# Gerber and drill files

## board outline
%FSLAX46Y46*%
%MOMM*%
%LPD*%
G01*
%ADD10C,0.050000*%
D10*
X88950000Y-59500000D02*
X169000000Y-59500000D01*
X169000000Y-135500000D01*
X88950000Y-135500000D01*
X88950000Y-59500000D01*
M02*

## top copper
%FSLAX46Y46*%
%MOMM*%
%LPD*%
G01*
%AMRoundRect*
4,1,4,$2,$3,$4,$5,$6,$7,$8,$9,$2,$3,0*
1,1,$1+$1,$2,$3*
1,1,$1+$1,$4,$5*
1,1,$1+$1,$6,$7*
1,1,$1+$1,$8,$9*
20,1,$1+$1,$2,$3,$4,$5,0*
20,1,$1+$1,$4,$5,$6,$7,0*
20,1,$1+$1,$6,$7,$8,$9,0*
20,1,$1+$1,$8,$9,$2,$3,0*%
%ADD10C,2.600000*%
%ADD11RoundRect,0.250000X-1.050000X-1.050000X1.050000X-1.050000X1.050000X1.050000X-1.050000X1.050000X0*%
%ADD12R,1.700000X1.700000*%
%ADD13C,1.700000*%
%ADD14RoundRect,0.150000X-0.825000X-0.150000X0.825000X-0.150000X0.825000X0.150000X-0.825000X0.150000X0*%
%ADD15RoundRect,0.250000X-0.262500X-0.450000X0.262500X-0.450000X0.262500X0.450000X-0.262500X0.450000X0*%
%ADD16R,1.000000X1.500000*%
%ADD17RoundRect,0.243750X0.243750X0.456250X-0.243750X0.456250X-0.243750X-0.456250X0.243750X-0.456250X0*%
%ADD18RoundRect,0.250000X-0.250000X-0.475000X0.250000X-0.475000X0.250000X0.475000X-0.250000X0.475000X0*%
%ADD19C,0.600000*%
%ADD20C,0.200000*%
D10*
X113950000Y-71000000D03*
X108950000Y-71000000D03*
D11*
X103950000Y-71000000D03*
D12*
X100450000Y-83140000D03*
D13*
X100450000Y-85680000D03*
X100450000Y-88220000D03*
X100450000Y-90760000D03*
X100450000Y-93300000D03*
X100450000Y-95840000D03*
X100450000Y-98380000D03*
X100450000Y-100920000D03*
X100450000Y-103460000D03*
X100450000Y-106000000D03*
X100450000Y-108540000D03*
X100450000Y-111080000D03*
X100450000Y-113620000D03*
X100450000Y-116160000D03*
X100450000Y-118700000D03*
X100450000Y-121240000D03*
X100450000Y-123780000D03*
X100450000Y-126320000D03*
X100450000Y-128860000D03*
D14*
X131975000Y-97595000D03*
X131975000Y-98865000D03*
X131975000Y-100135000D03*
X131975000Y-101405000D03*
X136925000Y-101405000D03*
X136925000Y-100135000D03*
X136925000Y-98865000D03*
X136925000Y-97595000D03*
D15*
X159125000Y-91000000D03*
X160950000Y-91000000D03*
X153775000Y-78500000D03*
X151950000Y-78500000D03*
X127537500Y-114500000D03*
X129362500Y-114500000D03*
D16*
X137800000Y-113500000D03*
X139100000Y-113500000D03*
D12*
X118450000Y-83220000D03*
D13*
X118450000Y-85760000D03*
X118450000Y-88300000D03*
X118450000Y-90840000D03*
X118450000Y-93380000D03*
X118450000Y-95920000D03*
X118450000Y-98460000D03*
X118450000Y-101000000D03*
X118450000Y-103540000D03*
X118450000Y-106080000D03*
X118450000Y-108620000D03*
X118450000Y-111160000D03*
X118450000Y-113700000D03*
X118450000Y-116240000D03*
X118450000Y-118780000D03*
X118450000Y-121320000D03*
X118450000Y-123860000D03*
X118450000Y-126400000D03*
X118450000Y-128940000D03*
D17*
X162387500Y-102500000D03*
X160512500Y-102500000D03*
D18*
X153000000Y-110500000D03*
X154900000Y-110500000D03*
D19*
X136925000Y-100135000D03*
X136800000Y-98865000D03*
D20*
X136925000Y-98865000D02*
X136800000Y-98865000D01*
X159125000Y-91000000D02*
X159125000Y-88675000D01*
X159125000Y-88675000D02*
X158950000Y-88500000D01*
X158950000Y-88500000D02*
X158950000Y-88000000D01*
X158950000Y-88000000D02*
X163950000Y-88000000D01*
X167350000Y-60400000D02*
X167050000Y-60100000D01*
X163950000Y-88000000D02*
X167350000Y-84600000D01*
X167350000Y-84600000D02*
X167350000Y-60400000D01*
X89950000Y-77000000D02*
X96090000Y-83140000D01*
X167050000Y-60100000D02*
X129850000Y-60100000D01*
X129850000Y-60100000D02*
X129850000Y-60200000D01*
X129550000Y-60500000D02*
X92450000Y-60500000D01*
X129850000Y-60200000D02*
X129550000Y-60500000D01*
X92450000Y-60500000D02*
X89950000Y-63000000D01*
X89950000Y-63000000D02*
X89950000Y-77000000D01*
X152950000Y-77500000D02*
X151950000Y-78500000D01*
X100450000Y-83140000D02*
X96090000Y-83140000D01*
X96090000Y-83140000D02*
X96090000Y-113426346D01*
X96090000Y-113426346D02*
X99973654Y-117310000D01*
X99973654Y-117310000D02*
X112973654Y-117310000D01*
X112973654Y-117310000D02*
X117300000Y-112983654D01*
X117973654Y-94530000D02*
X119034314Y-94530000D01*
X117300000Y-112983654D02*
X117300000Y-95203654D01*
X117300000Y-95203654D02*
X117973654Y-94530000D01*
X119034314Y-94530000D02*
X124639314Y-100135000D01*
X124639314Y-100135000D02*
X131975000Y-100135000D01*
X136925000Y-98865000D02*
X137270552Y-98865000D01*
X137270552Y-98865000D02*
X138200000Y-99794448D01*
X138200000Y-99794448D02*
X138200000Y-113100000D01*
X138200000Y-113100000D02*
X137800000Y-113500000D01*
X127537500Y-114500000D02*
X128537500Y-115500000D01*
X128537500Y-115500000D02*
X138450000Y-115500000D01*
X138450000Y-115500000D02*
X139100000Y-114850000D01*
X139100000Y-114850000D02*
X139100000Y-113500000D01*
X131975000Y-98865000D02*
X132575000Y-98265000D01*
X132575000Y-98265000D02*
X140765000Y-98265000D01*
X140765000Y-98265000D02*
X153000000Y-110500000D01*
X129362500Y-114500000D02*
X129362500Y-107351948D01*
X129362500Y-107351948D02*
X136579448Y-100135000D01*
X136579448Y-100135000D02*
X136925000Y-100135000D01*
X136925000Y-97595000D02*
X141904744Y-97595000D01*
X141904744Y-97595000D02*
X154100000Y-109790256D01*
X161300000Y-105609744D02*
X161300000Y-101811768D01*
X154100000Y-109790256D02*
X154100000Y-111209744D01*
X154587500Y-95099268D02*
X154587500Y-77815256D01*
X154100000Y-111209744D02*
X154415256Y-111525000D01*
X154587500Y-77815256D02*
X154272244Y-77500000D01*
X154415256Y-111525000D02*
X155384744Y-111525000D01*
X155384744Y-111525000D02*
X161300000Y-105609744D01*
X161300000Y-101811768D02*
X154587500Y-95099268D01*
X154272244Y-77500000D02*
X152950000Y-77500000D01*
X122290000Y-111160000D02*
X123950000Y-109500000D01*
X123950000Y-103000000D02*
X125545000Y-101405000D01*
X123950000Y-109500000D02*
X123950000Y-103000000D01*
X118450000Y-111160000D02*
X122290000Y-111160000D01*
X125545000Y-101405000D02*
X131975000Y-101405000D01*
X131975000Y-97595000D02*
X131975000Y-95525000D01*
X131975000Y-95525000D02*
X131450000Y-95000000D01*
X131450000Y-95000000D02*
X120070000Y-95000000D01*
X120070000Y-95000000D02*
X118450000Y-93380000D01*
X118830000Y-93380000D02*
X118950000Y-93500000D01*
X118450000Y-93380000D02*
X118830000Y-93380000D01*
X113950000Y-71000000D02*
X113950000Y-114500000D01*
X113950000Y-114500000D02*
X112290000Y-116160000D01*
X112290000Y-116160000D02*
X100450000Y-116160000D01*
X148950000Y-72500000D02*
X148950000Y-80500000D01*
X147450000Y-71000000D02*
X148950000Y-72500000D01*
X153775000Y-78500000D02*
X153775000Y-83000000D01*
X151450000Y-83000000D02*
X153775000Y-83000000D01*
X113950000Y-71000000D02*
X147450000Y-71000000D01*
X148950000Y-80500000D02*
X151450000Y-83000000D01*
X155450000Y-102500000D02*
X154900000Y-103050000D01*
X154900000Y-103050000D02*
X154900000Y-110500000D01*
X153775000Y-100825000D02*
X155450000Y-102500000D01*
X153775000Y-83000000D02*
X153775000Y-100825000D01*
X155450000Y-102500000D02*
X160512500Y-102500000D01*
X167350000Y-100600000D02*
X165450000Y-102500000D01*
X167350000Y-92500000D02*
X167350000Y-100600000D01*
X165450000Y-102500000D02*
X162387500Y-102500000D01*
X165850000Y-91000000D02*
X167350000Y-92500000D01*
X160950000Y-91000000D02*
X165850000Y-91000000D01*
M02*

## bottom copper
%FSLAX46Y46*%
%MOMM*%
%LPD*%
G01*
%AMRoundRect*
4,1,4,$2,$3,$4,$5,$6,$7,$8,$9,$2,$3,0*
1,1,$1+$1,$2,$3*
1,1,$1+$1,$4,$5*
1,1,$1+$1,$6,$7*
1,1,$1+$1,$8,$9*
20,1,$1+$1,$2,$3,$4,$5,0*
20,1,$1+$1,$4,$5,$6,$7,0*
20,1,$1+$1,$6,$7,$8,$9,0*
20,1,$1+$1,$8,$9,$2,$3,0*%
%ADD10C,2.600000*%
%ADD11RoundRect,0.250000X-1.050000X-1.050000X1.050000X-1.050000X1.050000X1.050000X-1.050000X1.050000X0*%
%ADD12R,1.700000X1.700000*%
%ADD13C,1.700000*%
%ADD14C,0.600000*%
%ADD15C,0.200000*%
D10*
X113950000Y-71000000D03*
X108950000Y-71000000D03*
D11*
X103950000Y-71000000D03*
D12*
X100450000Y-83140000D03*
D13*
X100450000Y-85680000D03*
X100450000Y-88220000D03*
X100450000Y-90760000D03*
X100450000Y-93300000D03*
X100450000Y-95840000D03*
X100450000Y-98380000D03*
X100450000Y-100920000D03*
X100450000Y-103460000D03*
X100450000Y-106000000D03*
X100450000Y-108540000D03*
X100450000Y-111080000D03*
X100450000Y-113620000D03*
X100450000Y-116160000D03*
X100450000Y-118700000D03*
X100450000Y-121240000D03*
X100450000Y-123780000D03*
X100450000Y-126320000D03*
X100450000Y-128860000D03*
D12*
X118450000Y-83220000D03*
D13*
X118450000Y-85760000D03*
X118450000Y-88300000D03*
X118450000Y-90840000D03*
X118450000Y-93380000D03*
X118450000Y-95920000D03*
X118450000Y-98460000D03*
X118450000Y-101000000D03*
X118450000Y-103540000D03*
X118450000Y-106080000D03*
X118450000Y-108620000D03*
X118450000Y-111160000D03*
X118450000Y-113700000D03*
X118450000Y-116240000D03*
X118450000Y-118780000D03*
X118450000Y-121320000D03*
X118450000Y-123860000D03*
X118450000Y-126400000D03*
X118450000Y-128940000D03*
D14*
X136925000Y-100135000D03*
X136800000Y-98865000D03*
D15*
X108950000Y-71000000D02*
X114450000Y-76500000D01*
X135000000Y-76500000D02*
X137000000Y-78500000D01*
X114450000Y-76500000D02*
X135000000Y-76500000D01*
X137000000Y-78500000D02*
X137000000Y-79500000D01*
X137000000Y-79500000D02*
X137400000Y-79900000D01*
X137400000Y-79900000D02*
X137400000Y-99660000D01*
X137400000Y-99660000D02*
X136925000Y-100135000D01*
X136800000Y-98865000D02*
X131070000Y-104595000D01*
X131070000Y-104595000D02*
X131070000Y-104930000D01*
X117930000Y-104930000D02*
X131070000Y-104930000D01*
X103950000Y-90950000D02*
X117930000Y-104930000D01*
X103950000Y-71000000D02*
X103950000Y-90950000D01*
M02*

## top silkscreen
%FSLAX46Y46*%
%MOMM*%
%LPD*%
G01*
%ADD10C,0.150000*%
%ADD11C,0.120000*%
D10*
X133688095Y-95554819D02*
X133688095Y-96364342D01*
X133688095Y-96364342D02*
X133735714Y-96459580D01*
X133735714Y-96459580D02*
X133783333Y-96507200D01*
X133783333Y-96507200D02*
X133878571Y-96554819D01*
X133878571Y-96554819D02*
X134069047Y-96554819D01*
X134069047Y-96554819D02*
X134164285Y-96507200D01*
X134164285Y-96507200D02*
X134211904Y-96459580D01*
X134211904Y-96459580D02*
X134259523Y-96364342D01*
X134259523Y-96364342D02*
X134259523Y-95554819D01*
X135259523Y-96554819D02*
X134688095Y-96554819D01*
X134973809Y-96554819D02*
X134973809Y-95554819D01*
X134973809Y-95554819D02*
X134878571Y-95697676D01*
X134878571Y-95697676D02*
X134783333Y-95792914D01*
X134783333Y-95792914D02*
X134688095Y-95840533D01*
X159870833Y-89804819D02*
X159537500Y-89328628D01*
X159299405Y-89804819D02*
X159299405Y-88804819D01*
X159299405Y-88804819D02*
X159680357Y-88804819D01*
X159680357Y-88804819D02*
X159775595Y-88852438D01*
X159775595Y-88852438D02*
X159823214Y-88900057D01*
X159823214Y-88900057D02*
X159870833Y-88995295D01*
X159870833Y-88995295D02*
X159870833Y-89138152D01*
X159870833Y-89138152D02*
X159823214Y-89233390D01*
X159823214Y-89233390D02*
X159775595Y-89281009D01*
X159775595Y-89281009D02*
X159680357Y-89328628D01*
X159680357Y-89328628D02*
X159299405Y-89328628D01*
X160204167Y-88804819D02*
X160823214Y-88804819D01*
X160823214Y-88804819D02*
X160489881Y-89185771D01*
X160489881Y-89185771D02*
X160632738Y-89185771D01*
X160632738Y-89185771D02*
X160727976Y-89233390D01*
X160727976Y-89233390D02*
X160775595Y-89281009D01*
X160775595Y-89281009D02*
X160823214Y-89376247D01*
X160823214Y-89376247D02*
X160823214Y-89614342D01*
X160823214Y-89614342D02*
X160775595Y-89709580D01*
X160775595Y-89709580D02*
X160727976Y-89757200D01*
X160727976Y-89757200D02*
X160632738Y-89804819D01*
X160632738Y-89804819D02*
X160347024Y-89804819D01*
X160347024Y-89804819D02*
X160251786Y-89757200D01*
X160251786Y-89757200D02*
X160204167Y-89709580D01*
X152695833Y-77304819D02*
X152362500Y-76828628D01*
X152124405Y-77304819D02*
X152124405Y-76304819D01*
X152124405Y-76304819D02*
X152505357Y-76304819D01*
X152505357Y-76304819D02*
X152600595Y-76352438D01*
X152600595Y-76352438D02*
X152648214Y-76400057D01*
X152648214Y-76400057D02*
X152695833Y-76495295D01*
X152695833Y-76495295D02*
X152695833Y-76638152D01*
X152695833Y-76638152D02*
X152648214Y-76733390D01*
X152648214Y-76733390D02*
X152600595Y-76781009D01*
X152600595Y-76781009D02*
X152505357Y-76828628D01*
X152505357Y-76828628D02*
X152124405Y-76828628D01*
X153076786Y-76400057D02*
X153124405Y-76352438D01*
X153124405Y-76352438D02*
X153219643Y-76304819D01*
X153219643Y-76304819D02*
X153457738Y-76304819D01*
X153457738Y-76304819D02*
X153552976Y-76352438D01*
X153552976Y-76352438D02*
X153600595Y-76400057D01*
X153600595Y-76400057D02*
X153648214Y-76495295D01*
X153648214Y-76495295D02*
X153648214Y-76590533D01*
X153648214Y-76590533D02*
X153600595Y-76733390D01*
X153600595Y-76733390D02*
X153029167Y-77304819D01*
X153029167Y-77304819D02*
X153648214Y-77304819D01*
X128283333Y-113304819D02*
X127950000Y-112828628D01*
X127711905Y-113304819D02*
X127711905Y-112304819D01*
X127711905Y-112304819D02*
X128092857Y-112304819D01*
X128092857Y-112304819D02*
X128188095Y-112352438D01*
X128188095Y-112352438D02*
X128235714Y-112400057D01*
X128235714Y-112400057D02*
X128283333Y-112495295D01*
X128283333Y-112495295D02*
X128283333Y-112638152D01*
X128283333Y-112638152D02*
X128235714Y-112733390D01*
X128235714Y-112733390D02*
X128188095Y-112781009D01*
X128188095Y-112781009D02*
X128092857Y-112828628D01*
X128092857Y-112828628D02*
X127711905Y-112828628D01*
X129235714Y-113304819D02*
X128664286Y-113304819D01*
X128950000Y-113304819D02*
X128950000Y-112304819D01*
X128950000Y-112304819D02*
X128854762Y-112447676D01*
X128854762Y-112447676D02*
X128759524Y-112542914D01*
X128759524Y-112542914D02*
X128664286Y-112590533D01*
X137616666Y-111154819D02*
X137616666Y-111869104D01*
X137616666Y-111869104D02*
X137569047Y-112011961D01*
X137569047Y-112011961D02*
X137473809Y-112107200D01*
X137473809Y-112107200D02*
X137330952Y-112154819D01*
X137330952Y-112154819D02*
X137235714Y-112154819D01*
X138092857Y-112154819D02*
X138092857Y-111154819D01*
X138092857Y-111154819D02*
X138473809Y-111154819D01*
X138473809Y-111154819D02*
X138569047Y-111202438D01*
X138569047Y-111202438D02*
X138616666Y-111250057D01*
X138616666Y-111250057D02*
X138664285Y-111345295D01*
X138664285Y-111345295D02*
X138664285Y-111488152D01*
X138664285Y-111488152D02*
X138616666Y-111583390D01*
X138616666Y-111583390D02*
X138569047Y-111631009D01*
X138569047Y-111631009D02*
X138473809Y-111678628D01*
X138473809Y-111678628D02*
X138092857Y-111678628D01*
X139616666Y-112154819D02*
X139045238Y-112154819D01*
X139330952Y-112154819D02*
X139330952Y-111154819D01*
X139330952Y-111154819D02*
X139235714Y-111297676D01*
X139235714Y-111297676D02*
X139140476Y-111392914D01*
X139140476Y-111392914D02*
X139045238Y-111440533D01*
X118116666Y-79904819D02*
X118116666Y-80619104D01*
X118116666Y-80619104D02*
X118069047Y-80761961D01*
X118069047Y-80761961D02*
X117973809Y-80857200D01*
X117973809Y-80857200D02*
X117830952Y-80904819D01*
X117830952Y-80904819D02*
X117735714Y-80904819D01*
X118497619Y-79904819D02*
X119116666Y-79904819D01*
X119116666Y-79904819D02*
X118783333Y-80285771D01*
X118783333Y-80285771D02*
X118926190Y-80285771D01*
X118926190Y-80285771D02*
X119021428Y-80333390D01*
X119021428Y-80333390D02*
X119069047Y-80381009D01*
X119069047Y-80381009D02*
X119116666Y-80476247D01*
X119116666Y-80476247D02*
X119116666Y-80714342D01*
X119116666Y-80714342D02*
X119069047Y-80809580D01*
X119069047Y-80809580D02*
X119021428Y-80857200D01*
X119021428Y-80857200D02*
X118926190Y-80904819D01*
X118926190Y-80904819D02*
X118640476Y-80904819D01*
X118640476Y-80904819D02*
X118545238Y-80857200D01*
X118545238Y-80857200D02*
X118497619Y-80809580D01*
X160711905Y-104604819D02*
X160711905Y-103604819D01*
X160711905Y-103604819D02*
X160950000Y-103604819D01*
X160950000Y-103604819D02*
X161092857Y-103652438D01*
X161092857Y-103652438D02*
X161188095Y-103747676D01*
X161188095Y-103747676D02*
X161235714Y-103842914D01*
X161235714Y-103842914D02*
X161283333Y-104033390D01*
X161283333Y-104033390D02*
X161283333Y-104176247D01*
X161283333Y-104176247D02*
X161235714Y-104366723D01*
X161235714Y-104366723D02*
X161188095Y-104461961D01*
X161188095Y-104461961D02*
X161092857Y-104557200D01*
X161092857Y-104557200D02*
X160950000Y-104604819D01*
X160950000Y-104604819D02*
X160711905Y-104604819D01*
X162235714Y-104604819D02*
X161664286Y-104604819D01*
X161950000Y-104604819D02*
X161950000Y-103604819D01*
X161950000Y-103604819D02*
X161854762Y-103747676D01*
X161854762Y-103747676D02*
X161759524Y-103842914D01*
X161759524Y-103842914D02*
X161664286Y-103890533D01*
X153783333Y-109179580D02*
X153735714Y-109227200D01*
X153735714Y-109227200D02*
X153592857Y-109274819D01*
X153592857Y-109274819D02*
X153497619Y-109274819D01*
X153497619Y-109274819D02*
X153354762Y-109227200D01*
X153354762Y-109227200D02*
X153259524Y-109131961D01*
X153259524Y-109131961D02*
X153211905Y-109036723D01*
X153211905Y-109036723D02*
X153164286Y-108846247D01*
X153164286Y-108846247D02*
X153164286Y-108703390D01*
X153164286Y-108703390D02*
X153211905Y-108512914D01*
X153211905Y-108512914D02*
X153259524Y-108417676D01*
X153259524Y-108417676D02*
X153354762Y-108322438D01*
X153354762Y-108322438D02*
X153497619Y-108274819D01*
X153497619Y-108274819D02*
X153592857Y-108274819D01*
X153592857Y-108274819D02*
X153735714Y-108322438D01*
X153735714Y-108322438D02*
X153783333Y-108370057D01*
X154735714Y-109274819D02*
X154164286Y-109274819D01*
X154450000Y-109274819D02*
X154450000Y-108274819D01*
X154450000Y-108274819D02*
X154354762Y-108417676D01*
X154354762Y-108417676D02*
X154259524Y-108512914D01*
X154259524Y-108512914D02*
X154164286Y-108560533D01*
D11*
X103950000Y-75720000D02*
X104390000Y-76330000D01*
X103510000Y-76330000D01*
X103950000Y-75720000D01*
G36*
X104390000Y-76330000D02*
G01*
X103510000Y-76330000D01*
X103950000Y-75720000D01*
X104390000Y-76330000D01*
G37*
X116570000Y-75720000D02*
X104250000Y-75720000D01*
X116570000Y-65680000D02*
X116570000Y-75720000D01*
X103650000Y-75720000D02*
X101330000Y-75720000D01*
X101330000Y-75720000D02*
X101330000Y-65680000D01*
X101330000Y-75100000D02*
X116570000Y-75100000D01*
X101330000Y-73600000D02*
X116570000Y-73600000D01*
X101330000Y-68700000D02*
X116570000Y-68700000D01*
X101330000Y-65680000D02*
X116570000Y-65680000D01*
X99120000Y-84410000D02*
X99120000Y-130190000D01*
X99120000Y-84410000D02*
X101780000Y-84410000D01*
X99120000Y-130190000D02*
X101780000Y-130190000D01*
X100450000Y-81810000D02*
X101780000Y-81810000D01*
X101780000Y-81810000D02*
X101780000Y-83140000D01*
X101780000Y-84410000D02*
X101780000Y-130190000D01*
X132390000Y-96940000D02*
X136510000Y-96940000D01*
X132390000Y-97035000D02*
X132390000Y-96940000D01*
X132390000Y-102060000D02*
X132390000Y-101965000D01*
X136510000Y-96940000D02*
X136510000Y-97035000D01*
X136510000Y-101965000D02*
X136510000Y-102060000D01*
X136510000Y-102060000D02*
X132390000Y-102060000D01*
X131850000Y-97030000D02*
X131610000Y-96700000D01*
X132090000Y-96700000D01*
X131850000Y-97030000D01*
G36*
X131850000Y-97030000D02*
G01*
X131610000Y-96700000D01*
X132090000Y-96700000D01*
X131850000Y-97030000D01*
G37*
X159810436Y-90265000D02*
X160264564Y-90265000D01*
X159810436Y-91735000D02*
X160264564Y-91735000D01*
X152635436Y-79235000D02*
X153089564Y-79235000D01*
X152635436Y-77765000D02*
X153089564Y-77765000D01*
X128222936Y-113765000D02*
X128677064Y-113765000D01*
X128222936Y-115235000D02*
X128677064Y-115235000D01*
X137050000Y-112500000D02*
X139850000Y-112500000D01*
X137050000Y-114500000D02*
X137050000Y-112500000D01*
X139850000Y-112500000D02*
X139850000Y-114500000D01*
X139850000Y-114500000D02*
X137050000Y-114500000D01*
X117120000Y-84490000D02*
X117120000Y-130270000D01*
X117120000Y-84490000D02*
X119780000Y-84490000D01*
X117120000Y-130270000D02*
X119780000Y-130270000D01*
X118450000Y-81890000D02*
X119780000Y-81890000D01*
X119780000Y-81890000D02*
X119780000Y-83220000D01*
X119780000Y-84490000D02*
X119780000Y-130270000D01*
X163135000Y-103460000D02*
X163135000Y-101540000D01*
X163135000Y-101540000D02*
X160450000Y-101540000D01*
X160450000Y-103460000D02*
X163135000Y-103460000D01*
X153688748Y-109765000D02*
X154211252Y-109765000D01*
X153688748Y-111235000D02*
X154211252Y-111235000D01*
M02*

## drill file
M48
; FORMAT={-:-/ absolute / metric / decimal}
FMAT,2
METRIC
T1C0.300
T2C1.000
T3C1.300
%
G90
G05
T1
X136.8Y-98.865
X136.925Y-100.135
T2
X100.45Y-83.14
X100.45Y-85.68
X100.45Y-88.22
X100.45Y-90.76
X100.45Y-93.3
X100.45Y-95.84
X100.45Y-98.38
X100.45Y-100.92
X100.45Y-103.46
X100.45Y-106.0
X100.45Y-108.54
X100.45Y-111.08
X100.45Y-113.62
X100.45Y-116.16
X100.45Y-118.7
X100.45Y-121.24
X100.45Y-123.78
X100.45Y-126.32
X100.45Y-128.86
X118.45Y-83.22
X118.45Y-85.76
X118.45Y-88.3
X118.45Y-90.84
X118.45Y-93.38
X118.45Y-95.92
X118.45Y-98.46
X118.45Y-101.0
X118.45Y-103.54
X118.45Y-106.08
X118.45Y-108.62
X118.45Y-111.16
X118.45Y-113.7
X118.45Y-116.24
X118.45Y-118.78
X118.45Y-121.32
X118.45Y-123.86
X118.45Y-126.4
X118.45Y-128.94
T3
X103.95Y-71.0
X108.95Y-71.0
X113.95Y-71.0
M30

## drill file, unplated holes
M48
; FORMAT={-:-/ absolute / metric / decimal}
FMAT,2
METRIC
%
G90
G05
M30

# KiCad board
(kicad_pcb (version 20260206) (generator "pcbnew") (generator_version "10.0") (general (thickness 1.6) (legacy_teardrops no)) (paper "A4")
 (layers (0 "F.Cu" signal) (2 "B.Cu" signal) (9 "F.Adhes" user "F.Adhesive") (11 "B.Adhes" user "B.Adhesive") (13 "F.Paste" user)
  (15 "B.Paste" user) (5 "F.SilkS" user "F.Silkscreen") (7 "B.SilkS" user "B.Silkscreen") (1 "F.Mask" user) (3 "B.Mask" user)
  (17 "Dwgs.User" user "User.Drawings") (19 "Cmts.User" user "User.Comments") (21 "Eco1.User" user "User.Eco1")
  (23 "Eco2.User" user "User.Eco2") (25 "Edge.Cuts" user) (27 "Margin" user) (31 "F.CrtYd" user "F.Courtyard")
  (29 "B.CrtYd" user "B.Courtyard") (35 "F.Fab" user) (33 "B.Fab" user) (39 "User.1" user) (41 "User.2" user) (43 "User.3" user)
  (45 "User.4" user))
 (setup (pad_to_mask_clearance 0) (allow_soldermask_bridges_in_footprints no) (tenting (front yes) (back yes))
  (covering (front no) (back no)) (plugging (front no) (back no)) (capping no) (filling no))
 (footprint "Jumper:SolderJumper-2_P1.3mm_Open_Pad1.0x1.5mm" (layer "F.Cu") (at 138.45 113.5)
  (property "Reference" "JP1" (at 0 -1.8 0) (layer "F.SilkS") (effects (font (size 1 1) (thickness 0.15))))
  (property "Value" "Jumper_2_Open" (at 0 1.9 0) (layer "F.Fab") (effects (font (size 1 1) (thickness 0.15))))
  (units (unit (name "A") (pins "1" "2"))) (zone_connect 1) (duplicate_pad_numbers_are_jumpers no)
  (fp_line (start -1.4 -1) (end 1.4 -1) (stroke (width 0.12) (type solid)) (layer "F.SilkS"))
  (fp_line (start -1.4 1) (end -1.4 -1) (stroke (width 0.12) (type solid)) (layer "F.SilkS"))
  (fp_line (start 1.4 -1) (end 1.4 1) (stroke (width 0.12) (type solid)) (layer "F.SilkS"))
  (fp_line (start 1.4 1) (end -1.4 1) (stroke (width 0.12) (type solid)) (layer "F.SilkS"))
  (pad "1" smd rect (at -0.65 0) (size 1 1.5) (layers "F.Cu" "F.Mask") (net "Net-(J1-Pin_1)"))
  (pad "2" smd rect (at 0.65 0) (size 1 1.5) (layers "F.Cu" "F.Mask") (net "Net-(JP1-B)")))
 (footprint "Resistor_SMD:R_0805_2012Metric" (layer "F.Cu") (at 152.8625 78.5)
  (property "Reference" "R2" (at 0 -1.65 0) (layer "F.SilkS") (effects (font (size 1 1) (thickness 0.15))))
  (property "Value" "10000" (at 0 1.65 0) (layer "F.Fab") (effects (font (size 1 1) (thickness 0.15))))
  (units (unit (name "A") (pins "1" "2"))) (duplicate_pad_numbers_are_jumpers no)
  (fp_line (start -0.227064 -0.735) (end 0.227064 -0.735) (stroke (width 0.12) (type solid)) (layer "F.SilkS"))
  (fp_line (start -0.227064 0.735) (end 0.227064 0.735) (stroke (width 0.12) (type solid)) (layer "F.SilkS"))
  (pad "1" smd roundrect (at -0.9125 0) (size 1.025 1.4) (layers "F.Cu" "F.Mask" "F.Paste") (roundrect_rratio 0.243902) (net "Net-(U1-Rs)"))
  (pad "2" smd roundrect (at 0.9125 0) (size 1.025 1.4) (layers "F.Cu" "F.Mask" "F.Paste") (roundrect_rratio 0.243902) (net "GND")))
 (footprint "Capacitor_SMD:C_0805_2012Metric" (layer "F.Cu") (at 153.95 110.5)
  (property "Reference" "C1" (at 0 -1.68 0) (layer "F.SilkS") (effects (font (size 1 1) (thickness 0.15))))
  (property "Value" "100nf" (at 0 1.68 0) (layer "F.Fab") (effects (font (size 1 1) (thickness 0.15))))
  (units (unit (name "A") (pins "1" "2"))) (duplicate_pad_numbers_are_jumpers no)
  (fp_line (start -0.261252 -0.735) (end 0.261252 -0.735) (stroke (width 0.12) (type solid)) (layer "F.SilkS"))
  (fp_line (start -0.261252 0.735) (end 0.261252 0.735) (stroke (width 0.12) (type solid)) (layer "F.SilkS"))
  (pad "1" smd roundrect (at -0.95 0) (size 1 1.45) (layers "F.Cu" "F.Mask" "F.Paste") (roundrect_rratio 0.25) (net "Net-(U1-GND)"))
  (pad "2" smd roundrect (at 0.95 0) (size 1 1.45) (layers "F.Cu" "F.Mask" "F.Paste") (roundrect_rratio 0.25) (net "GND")))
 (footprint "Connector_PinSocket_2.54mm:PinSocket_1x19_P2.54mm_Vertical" (layer "F.Cu") (at 100.45 83.14)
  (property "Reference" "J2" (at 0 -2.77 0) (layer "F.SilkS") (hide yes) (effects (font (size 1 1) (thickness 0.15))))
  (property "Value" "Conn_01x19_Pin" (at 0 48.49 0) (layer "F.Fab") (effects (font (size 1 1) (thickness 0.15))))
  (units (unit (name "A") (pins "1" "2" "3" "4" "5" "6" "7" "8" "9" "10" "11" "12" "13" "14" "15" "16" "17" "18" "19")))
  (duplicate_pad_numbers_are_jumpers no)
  (fp_line (start -1.33 1.27) (end -1.33 47.05) (stroke (width 0.12) (type solid)) (layer "F.SilkS"))
  (fp_line (start -1.33 1.27) (end 1.33 1.27) (stroke (width 0.12) (type solid)) (layer "F.SilkS"))
  (fp_line (start -1.33 47.05) (end 1.33 47.05) (stroke (width 0.12) (type solid)) (layer "F.SilkS"))
  (fp_line (start 0 -1.33) (end 1.33 -1.33) (stroke (width 0.12) (type solid)) (layer "F.SilkS"))
  (fp_line (start 1.33 -1.33) (end 1.33 0) (stroke (width 0.12) (type solid)) (layer "F.SilkS"))
  (fp_line (start 1.33 1.27) (end 1.33 47.05) (stroke (width 0.12) (type solid)) (layer "F.SilkS"))
  (pad "1" thru_hole rect (at 0 0) (size 1.7 1.7) (drill 1) (layers "*.Cu" "*.Mask") (remove_unused_layers no) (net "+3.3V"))
  (pad "2" thru_hole circle (at 0 2.54) (size 1.7 1.7) (drill 1) (layers "*.Cu" "*.Mask") (remove_unused_layers no)
   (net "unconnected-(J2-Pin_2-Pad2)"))
  (pad "3" thru_hole circle (at 0 5.08) (size 1.7 1.7) (drill 1) (layers "*.Cu" "*.Mask") (remove_unused_layers no)
   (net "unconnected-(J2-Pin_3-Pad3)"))
  (pad "4" thru_hole circle (at 0 7.62) (size 1.7 1.7) (drill 1) (layers "*.Cu" "*.Mask") (remove_unused_layers no)
   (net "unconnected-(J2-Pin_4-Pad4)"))
  (pad "5" thru_hole circle (at 0 10.16) (size 1.7 1.7) (drill 1) (layers "*.Cu" "*.Mask") (remove_unused_layers no)
   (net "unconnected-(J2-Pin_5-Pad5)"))
  (pad "6" thru_hole circle (at 0 12.7) (size 1.7 1.7) (drill 1) (layers "*.Cu" "*.Mask") (remove_unused_layers no)
   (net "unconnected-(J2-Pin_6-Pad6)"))
  (pad "7" thru_hole circle (at 0 15.24) (size 1.7 1.7) (drill 1) (layers "*.Cu" "*.Mask") (remove_unused_layers no)
   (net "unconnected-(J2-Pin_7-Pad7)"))
  (pad "8" thru_hole circle (at 0 17.78) (size 1.7 1.7) (drill 1) (layers "*.Cu" "*.Mask") (remove_unused_layers no)
   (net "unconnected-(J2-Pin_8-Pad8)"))
  (pad "9" thru_hole circle (at 0 20.32) (size 1.7 1.7) (drill 1) (layers "*.Cu" "*.Mask") (remove_unused_layers no)
   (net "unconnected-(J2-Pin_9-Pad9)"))
  (pad "10" thru_hole circle (at 0 22.86) (size 1.7 1.7) (drill 1) (layers "*.Cu" "*.Mask") (remove_unused_layers no)
   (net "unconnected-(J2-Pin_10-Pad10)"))
  (pad "11" thru_hole circle (at 0 25.4) (size 1.7 1.7) (drill 1) (layers "*.Cu" "*.Mask") (remove_unused_layers no)
   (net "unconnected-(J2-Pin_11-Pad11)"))
  (pad "12" thru_hole circle (at 0 27.94) (size 1.7 1.7) (drill 1) (layers "*.Cu" "*.Mask") (remove_unused_layers no)
   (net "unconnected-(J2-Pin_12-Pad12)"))
  (pad "13" thru_hole circle (at 0 30.48) (size 1.7 1.7) (drill 1) (layers "*.Cu" "*.Mask") (remove_unused_layers no)
   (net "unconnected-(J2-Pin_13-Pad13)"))
  (pad "14" thru_hole circle (at 0 33.02) (size 1.7 1.7) (drill 1) (layers "*.Cu" "*.Mask") (remove_unused_layers no) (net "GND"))
  (pad "15" thru_hole circle (at 0 35.56) (size 1.7 1.7) (drill 1) (layers "*.Cu" "*.Mask") (remove_unused_layers no)
   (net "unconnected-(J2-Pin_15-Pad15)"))
  (pad "16" thru_hole circle (at 0 38.1) (size 1.7 1.7) (drill 1) (layers "*.Cu" "*.Mask") (remove_unused_layers no)
   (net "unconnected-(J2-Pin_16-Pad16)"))
  (pad "17" thru_hole circle (at 0 40.64) (size 1.7 1.7) (drill 1) (layers "*.Cu" "*.Mask") (remove_unused_layers no)
   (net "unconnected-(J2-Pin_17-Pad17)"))
  (pad "18" thru_hole circle (at 0 43.18) (size 1.7 1.7) (drill 1) (layers "*.Cu" "*.Mask") (remove_unused_layers no)
   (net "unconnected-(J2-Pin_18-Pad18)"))
  (pad "19" thru_hole circle (at 0 45.72) (size 1.7 1.7) (drill 1) (layers "*.Cu" "*.Mask") (remove_unused_layers no)
   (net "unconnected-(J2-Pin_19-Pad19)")))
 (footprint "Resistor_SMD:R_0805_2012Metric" (layer "F.Cu") (at 128.45 114.5)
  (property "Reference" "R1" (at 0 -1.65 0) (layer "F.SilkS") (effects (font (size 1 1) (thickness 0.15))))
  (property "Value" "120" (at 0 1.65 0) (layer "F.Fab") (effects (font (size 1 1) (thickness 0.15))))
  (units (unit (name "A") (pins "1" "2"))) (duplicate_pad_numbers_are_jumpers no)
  (fp_line (start -0.227064 -0.735) (end 0.227064 -0.735) (stroke (width 0.12) (type solid)) (layer "F.SilkS"))
  (fp_line (start -0.227064 0.735) (end 0.227064 0.735) (stroke (width 0.12) (type solid)) (layer "F.SilkS"))
  (pad "1" smd roundrect (at -0.9125 0) (size 1.025 1.4) (layers "F.Cu" "F.Mask" "F.Paste") (roundrect_rratio 0.243902) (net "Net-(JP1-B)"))
  (pad "2" smd roundrect (at 0.9125 0) (size 1.025 1.4) (layers "F.Cu" "F.Mask" "F.Paste") (roundrect_rratio 0.243902)
   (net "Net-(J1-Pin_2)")))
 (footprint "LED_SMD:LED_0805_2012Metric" (layer "F.Cu") (at 161.45 102.5 180)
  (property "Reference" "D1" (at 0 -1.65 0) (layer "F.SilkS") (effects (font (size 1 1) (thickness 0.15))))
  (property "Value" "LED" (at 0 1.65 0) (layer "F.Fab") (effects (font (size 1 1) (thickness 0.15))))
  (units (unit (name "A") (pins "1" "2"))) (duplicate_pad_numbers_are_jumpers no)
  (fp_line (start 1 -0.96) (end -1.685 -0.96) (stroke (width 0.12) (type solid)) (layer "F.SilkS"))
  (fp_line (start -1.685 0.96) (end 1 0.96) (stroke (width 0.12) (type solid)) (layer "F.SilkS"))
  (fp_line (start -1.685 -0.96) (end -1.685 0.96) (stroke (width 0.12) (type solid)) (layer "F.SilkS"))
  (pad "1" smd roundrect (at -0.9375 0 180) (size 0.975 1.4) (layers "F.Cu" "F.Mask" "F.Paste") (roundrect_rratio 0.25) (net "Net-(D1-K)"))
  (pad "2" smd roundrect (at 0.9375 0 180) (size 0.975 1.4) (layers "F.Cu" "F.Mask" "F.Paste") (roundrect_rratio 0.25) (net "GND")))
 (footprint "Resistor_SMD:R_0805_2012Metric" (layer "F.Cu") (at 160.0375 91)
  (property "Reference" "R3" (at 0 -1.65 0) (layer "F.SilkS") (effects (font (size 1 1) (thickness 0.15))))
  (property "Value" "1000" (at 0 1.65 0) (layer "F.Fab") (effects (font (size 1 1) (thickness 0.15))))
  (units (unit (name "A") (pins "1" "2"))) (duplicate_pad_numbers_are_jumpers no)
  (fp_line (start -0.227064 -0.735) (end 0.227064 -0.735) (stroke (width 0.12) (type solid)) (layer "F.SilkS"))
  (fp_line (start -0.227064 0.735) (end 0.227064 0.735) (stroke (width 0.12) (type solid)) (layer "F.SilkS"))
  (pad "1" smd roundrect (at -0.9125 0) (size 1.025 1.4) (layers "F.Cu" "F.Mask" "F.Paste") (roundrect_rratio 0.243902) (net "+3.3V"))
  (pad "2" smd roundrect (at 0.9125 0) (size 1.025 1.4) (layers "F.Cu" "F.Mask" "F.Paste") (roundrect_rratio 0.243902) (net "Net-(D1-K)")))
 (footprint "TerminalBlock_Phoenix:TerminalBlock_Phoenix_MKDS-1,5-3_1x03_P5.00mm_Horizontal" (layer "F.Cu") (at 103.95 71)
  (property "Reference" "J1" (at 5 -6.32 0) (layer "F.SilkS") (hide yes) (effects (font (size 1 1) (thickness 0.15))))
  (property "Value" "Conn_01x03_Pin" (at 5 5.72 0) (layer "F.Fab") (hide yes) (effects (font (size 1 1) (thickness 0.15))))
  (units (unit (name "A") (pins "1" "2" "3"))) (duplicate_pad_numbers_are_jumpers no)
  (fp_line (start -2.62 -5.32) (end 12.62 -5.32) (stroke (width 0.12) (type solid)) (layer "F.SilkS"))
  (fp_line (start -2.62 -2.3) (end 12.62 -2.3) (stroke (width 0.12) (type solid)) (layer "F.SilkS"))
  (fp_line (start -2.62 2.6) (end 12.62 2.6) (stroke (width 0.12) (type solid)) (layer "F.SilkS"))
  (fp_line (start -2.62 4.1) (end 12.62 4.1) (stroke (width 0.12) (type solid)) (layer "F.SilkS"))
  (fp_line (start -2.62 4.72) (end -2.62 -5.32) (stroke (width 0.12) (type solid)) (layer "F.SilkS"))
  (fp_line (start -0.3 4.72) (end -2.62 4.72) (stroke (width 0.12) (type solid)) (layer "F.SilkS"))
  (fp_line (start 12.62 -5.32) (end 12.62 4.72) (stroke (width 0.12) (type solid)) (layer "F.SilkS"))
  (fp_line (start 12.62 4.72) (end 0.3 4.72) (stroke (width 0.12) (type solid)) (layer "F.SilkS"))
  (fp_poly (pts (xy 0 4.72) (xy 0.44 5.33) (xy -0.44 5.33)) (stroke (width 0.12) (type solid)) (fill yes) (layer "F.SilkS"))
  (pad "1" thru_hole roundrect (at 0 0) (size 2.6 2.6) (drill 1.3) (layers "*.Cu" "*.Mask") (remove_unused_layers no)
   (roundrect_rratio 0.096154) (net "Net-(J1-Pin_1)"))
  (pad "2" thru_hole circle (at 5 0) (size 2.6 2.6) (drill 1.3) (layers "*.Cu" "*.Mask") (remove_unused_layers no) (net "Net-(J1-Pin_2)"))
  (pad "3" thru_hole circle (at 10 0) (size 2.6 2.6) (drill 1.3) (layers "*.Cu" "*.Mask") (remove_unused_layers no) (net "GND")))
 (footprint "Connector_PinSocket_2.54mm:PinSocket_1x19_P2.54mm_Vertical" (layer "F.Cu") (at 118.45 83.22)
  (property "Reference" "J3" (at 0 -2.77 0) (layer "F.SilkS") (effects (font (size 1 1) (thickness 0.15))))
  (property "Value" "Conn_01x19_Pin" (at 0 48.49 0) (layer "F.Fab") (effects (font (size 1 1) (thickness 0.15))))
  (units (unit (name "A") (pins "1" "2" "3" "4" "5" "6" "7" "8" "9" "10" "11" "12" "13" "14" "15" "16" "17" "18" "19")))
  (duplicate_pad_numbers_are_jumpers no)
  (fp_line (start -1.33 1.27) (end -1.33 47.05) (stroke (width 0.12) (type solid)) (layer "F.SilkS"))
  (fp_line (start -1.33 1.27) (end 1.33 1.27) (stroke (width 0.12) (type solid)) (layer "F.SilkS"))
  (fp_line (start -1.33 47.05) (end 1.33 47.05) (stroke (width 0.12) (type solid)) (layer "F.SilkS"))
  (fp_line (start 0 -1.33) (end 1.33 -1.33) (stroke (width 0.12) (type solid)) (layer "F.SilkS"))
  (fp_line (start 1.33 -1.33) (end 1.33 0) (stroke (width 0.12) (type solid)) (layer "F.SilkS"))
  (fp_line (start 1.33 1.27) (end 1.33 47.05) (stroke (width 0.12) (type solid)) (layer "F.SilkS"))
  (pad "1" thru_hole rect (at 0 0) (size 1.7 1.7) (drill 1) (layers "*.Cu" "*.Mask") (remove_unused_layers no)
   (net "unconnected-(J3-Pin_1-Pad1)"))
  (pad "2" thru_hole circle (at 0 2.54) (size 1.7 1.7) (drill 1) (layers "*.Cu" "*.Mask") (remove_unused_layers no)
   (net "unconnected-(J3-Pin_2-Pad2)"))
  (pad "3" thru_hole circle (at 0 5.08) (size 1.7 1.7) (drill 1) (layers "*.Cu" "*.Mask") (remove_unused_layers no)
   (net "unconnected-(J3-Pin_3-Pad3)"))
  (pad "4" thru_hole circle (at 0 7.62) (size 1.7 1.7) (drill 1) (layers "*.Cu" "*.Mask") (remove_unused_layers no)
   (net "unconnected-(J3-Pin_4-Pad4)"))
  (pad "5" thru_hole circle (at 0 10.16) (size 1.7 1.7) (drill 1) (layers "*.Cu" "*.Mask") (remove_unused_layers no) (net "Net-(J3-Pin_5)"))
  (pad "6" thru_hole circle (at 0 12.7) (size 1.7 1.7) (drill 1) (layers "*.Cu" "*.Mask") (remove_unused_layers no)
   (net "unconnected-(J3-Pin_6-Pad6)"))
  (pad "7" thru_hole circle (at 0 15.24) (size 1.7 1.7) (drill 1) (layers "*.Cu" "*.Mask") (remove_unused_layers no)
   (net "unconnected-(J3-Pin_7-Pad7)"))
  (pad "8" thru_hole circle (at 0 17.78) (size 1.7 1.7) (drill 1) (layers "*.Cu" "*.Mask") (remove_unused_layers no)
   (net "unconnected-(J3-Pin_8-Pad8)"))
  (pad "9" thru_hole circle (at 0 20.32) (size 1.7 1.7) (drill 1) (layers "*.Cu" "*.Mask") (remove_unused_layers no)
   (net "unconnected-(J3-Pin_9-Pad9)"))
  (pad "10" thru_hole circle (at 0 22.86) (size 1.7 1.7) (drill 1) (layers "*.Cu" "*.Mask") (remove_unused_layers no)
   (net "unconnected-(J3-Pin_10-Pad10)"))
  (pad "11" thru_hole circle (at 0 25.4) (size 1.7 1.7) (drill 1) (layers "*.Cu" "*.Mask") (remove_unused_layers no)
   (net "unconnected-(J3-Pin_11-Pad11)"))
  (pad "12" thru_hole circle (at 0 27.94) (size 1.7 1.7) (drill 1) (layers "*.Cu" "*.Mask") (remove_unused_layers no)
   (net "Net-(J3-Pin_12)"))
  (pad "13" thru_hole circle (at 0 30.48) (size 1.7 1.7) (drill 1) (layers "*.Cu" "*.Mask") (remove_unused_layers no)
   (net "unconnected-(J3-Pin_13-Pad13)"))
  (pad "14" thru_hole circle (at 0 33.02) (size 1.7 1.7) (drill 1) (layers "*.Cu" "*.Mask") (remove_unused_layers no)
   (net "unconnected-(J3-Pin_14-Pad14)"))
  (pad "15" thru_hole circle (at 0 35.56) (size 1.7 1.7) (drill 1) (layers "*.Cu" "*.Mask") (remove_unused_layers no)
   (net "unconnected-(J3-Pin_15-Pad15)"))
  (pad "16" thru_hole circle (at 0 38.1) (size 1.7 1.7) (drill 1) (layers "*.Cu" "*.Mask") (remove_unused_layers no)
   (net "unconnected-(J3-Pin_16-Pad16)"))
  (pad "17" thru_hole circle (at 0 40.64) (size 1.7 1.7) (drill 1) (layers "*.Cu" "*.Mask") (remove_unused_layers no)
   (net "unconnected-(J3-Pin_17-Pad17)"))
  (pad "18" thru_hole circle (at 0 43.18) (size 1.7 1.7) (drill 1) (layers "*.Cu" "*.Mask") (remove_unused_layers no)
   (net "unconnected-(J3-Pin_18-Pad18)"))
  (pad "19" thru_hole circle (at 0 45.72) (size 1.7 1.7) (drill 1) (layers "*.Cu" "*.Mask") (remove_unused_layers no)
   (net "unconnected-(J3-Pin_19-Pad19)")))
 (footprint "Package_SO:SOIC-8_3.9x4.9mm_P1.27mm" (layer "F.Cu") (at 134.45 99.5)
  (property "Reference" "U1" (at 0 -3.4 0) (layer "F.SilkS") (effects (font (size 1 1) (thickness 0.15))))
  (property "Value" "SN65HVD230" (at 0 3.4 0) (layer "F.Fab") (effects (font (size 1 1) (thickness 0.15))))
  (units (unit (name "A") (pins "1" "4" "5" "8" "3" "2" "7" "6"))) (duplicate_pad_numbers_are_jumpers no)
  (fp_line (start -2.06 -2.56) (end 2.06 -2.56) (stroke (width 0.12) (type solid)) (layer "F.SilkS"))
  (fp_line (start -2.06 -2.465) (end -2.06 -2.56) (stroke (width 0.12) (type solid)) (layer "F.SilkS"))
  (fp_line (start -2.06 2.56) (end -2.06 2.465) (stroke (width 0.12) (type solid)) (layer "F.SilkS"))
  (fp_line (start 2.06 -2.56) (end 2.06 -2.465) (stroke (width 0.12) (type solid)) (layer "F.SilkS"))
  (fp_line (start 2.06 2.465) (end 2.06 2.56) (stroke (width 0.12) (type solid)) (layer "F.SilkS"))
  (fp_line (start 2.06 2.56) (end -2.06 2.56) (stroke (width 0.12) (type solid)) (layer "F.SilkS"))
  (fp_poly (pts (xy -2.6 -2.47) (xy -2.84 -2.8) (xy -2.36 -2.8)) (stroke (width 0.12) (type solid)) (fill yes) (layer "F.SilkS"))
  (pad "1" smd roundrect (at -2.475 -1.905) (size 1.95 0.6) (layers "F.Cu" "F.Mask" "F.Paste") (roundrect_rratio 0.25)
   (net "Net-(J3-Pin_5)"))
  (pad "2" smd roundrect (at -2.475 -0.635) (size 1.95 0.6) (layers "F.Cu" "F.Mask" "F.Paste") (roundrect_rratio 0.25) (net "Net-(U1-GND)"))
  (pad "3" smd roundrect (at -2.475 0.635) (size 1.95 0.6) (layers "F.Cu" "F.Mask" "F.Paste") (roundrect_rratio 0.25) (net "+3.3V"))
  (pad "4" smd roundrect (at -2.475 1.905) (size 1.95 0.6) (layers "F.Cu" "F.Mask" "F.Paste") (roundrect_rratio 0.25)
   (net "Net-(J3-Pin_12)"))
  (pad "5" smd roundrect (at 2.475 1.905) (size 1.95 0.6) (layers "F.Cu" "F.Mask" "F.Paste") (roundrect_rratio 0.25)
   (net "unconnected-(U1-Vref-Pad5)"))
  (pad "6" smd roundrect (at 2.475 0.635) (size 1.95 0.6) (layers "F.Cu" "F.Mask" "F.Paste") (roundrect_rratio 0.25) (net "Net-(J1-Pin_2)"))
  (pad "7" smd roundrect (at 2.475 -0.635) (size 1.95 0.6) (layers "F.Cu" "F.Mask" "F.Paste") (roundrect_rratio 0.25) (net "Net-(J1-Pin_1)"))
  (pad "8" smd roundrect (at 2.475 -1.905) (size 1.95 0.6) (layers "F.Cu" "F.Mask" "F.Paste") (roundrect_rratio 0.25) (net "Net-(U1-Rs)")))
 (gr_rect (start 88.95 59.5) (end 169 135.5) (stroke (width 0.05) (type default)) (fill no) (layer "Edge.Cuts"))
 (segment (start 148.95 80.5) (end 151.45 83) (width 0.2) (layer "F.Cu") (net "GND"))
 (segment (start 113.95 71) (end 113.95 114.5) (width 0.2) (layer "F.Cu") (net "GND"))
 (segment (start 155.45 102.5) (end 154.9 103.05) (width 0.2) (layer "F.Cu") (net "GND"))
 (segment (start 153.775 78.5) (end 153.775 83) (width 0.2) (layer "F.Cu") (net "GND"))
 (segment (start 113.95 114.5) (end 112.29 116.16) (width 0.2) (layer "F.Cu") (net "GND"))
 (segment (start 155.45 102.5) (end 160.5125 102.5) (width 0.2) (layer "F.Cu") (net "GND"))
 (segment (start 154.9 103.05) (end 154.9 110.5) (width 0.2) (layer "F.Cu") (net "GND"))
 (segment (start 113.95 71) (end 147.45 71) (width 0.2) (layer "F.Cu") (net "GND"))
 (segment (start 153.775 83) (end 153.775 100.825) (width 0.2) (layer "F.Cu") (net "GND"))
 (segment (start 112.29 116.16) (end 100.45 116.16) (width 0.2) (layer "F.Cu") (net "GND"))
 (segment (start 151.45 83) (end 153.775 83) (width 0.2) (layer "F.Cu") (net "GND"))
 (segment (start 153.775 100.825) (end 155.45 102.5) (width 0.2) (layer "F.Cu") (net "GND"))
 (segment (start 147.45 71) (end 148.95 72.5) (width 0.2) (layer "F.Cu") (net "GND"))
 (segment (start 148.95 72.5) (end 148.95 80.5) (width 0.2) (layer "F.Cu") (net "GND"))
 (segment (start 140.765 98.265) (end 153 110.5) (width 0.2) (layer "F.Cu") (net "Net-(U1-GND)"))
 (segment (start 132.575 98.265) (end 140.765 98.265) (width 0.2) (layer "F.Cu") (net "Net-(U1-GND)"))
 (segment (start 131.975 98.865) (end 132.575 98.265) (width 0.2) (layer "F.Cu") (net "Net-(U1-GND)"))
 (segment (start 167.35 92.5) (end 167.35 100.6) (width 0.2) (layer "F.Cu") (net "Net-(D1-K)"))
 (segment (start 167.35 100.6) (end 165.45 102.5) (width 0.2) (layer "F.Cu") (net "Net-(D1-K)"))
 (segment (start 160.95 91) (end 165.85 91) (width 0.2) (layer "F.Cu") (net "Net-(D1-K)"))
 (segment (start 165.45 102.5) (end 162.3875 102.5) (width 0.2) (layer "F.Cu") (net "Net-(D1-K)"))
 (segment (start 165.85 91) (end 167.35 92.5) (width 0.2) (layer "F.Cu") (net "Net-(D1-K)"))
 (segment (start 136.579448 100.135) (end 136.925 100.135) (width 0.2) (layer "F.Cu") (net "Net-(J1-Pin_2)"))
 (segment (start 129.3625 114.5) (end 129.3625 107.351948) (width 0.2) (layer "F.Cu") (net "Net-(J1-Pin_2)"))
 (segment (start 129.3625 107.351948) (end 136.579448 100.135) (width 0.2) (layer "F.Cu") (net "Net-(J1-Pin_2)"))
 (via blind (at 136.925 100.135) (size 0.6) (drill 0.3) (layers "F.Cu" "B.Cu") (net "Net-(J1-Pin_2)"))
 (segment (start 108.95 71) (end 114.45 76.5) (width 0.2) (layer "B.Cu") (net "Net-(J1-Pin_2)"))
 (segment (start 137 78.5) (end 137 79.5) (width 0.2) (layer "B.Cu") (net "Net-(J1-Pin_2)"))
 (segment (start 135 76.5) (end 137 78.5) (width 0.2) (layer "B.Cu") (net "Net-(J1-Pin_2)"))
 (segment (start 137 79.5) (end 137.4 79.9) (width 0.2) (layer "B.Cu") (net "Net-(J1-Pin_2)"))
 (segment (start 137.4 99.66) (end 136.925 100.135) (width 0.2) (layer "B.Cu") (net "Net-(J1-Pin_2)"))
 (segment (start 137.4 79.9) (end 137.4 99.66) (width 0.2) (layer "B.Cu") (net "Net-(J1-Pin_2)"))
 (segment (start 114.45 76.5) (end 135 76.5) (width 0.2) (layer "B.Cu") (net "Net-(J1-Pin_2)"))
 (segment (start 136.925 98.865) (end 137.270552 98.865) (width 0.2) (layer "F.Cu") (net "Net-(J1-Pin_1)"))
 (segment (start 138.2 113.1) (end 137.8 113.5) (width 0.2) (layer "F.Cu") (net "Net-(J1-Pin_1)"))
 (segment (start 136.925 98.865) (end 136.8 98.865) (width 0.2) (layer "F.Cu") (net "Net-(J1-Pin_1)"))
 (segment (start 138.2 99.794448) (end 138.2 113.1) (width 0.2) (layer "F.Cu") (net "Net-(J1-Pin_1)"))
 (segment (start 137.270552 98.865) (end 138.2 99.794448) (width 0.2) (layer "F.Cu") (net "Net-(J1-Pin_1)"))
 (via blind (at 136.8 98.865) (size 0.6) (drill 0.3) (layers "F.Cu" "B.Cu") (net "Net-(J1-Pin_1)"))
 (segment (start 103.95 71) (end 103.95 90.95) (width 0.2) (layer "B.Cu") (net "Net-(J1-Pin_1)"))
 (segment (start 136.8 98.865) (end 131.07 104.595) (width 0.2) (layer "B.Cu") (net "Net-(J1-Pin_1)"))
 (segment (start 117.93 104.93) (end 131.07 104.93) (width 0.2) (layer "B.Cu") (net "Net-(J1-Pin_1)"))
 (segment (start 103.95 90.95) (end 117.93 104.93) (width 0.2) (layer "B.Cu") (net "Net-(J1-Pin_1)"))
 (segment (start 131.07 104.595) (end 131.07 104.93) (width 0.2) (layer "B.Cu") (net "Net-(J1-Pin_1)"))
 (segment (start 163.95 88) (end 167.35 84.6) (width 0.2) (layer "F.Cu") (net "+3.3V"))
 (segment (start 117.3 112.983654) (end 117.3 95.203654) (width 0.2) (layer "F.Cu") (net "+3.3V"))
 (segment (start 158.95 88) (end 163.95 88) (width 0.2) (layer "F.Cu") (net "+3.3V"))
 (segment (start 129.85 60.2) (end 129.55 60.5) (width 0.2) (layer "F.Cu") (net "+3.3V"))
 (segment (start 119.034314 94.53) (end 124.639314 100.135) (width 0.2) (layer "F.Cu") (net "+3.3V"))
 (segment (start 167.05 60.1) (end 129.85 60.1) (width 0.2) (layer "F.Cu") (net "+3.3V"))
 (segment (start 129.55 60.5) (end 92.45 60.5) (width 0.2) (layer "F.Cu") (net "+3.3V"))
 (segment (start 167.35 84.6) (end 167.35 60.4) (width 0.2) (layer "F.Cu") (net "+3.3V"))
 (segment (start 129.85 60.1) (end 129.85 60.2) (width 0.2) (layer "F.Cu") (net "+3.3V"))
 (segment (start 117.973654 94.53) (end 119.034314 94.53) (width 0.2) (layer "F.Cu") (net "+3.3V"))
 (segment (start 159.125 91) (end 159.125 88.675) (width 0.2) (layer "F.Cu") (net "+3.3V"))
 (segment (start 159.125 88.675) (end 158.95 88.5) (width 0.2) (layer "F.Cu") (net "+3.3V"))
 (segment (start 117.3 95.203654) (end 117.973654 94.53) (width 0.2) (layer "F.Cu") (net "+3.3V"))
 (segment (start 158.95 88.5) (end 158.95 88) (width 0.2) (layer "F.Cu") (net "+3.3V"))
 (segment (start 112.973654 117.31) (end 117.3 112.983654) (width 0.2) (layer "F.Cu") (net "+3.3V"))
 (segment (start 167.35 60.4) (end 167.05 60.1) (width 0.2) (layer "F.Cu") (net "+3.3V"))
 (segment (start 89.95 77) (end 96.09 83.14) (width 0.2) (layer "F.Cu") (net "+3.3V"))
 (segment (start 100.45 83.14) (end 96.09 83.14) (width 0.2) (layer "F.Cu") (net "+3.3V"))
 (segment (start 99.973654 117.31) (end 112.973654 117.31) (width 0.2) (layer "F.Cu") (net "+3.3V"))
 (segment (start 96.09 83.14) (end 96.09 113.426346) (width 0.2) (layer "F.Cu") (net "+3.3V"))
 (segment (start 124.639314 100.135) (end 131.975 100.135) (width 0.2) (layer "F.Cu") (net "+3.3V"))
 (segment (start 89.95 63) (end 89.95 77) (width 0.2) (layer "F.Cu") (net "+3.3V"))
 (segment (start 96.09 113.426346) (end 99.973654 117.31) (width 0.2) (layer "F.Cu") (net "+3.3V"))
 (segment (start 92.45 60.5) (end 89.95 63) (width 0.2) (layer "F.Cu") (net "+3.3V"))
 (segment (start 118.45 111.16) (end 122.29 111.16) (width 0.2) (layer "F.Cu") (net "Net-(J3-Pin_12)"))
 (segment (start 123.95 109.5) (end 123.95 103) (width 0.2) (layer "F.Cu") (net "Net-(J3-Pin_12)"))
 (segment (start 125.545 101.405) (end 131.975 101.405) (width 0.2) (layer "F.Cu") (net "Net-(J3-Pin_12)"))
 (segment (start 122.29 111.16) (end 123.95 109.5) (width 0.2) (layer "F.Cu") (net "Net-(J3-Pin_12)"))
 (segment (start 123.95 103) (end 125.545 101.405) (width 0.2) (layer "F.Cu") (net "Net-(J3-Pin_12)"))
 (segment (start 120.07 95) (end 118.45 93.38) (width 0.2) (layer "F.Cu") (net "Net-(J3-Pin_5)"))
 (segment (start 118.45 93.38) (end 118.83 93.38) (width 0.2) (layer "F.Cu") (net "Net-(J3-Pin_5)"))
 (segment (start 131.975 95.525) (end 131.45 95) (width 0.2) (layer "F.Cu") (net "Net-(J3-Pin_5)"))
 (segment (start 131.975 97.595) (end 131.975 95.525) (width 0.2) (layer "F.Cu") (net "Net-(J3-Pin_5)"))
 (segment (start 131.45 95) (end 120.07 95) (width 0.2) (layer "F.Cu") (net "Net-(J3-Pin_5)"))
 (segment (start 118.83 93.38) (end 118.95 93.5) (width 0.2) (layer "F.Cu") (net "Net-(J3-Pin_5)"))
 (segment (start 127.5375 114.5) (end 128.5375 115.5) (width 0.2) (layer "F.Cu") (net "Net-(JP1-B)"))
 (segment (start 138.45 115.5) (end 139.1 114.85) (width 0.2) (layer "F.Cu") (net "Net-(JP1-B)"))
 (segment (start 128.5375 115.5) (end 138.45 115.5) (width 0.2) (layer "F.Cu") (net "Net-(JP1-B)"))
 (segment (start 139.1 114.85) (end 139.1 113.5) (width 0.2) (layer "F.Cu") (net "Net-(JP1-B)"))
 (segment (start 141.904744 97.595) (end 154.1 109.790256) (width 0.2) (layer "F.Cu") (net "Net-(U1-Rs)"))
 (segment (start 154.5875 95.099268) (end 154.5875 77.815256) (width 0.2) (layer "F.Cu") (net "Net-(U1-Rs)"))
 (segment (start 161.3 101.811768) (end 154.5875 95.099268) (width 0.2) (layer "F.Cu") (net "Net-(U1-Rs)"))
 (segment (start 154.272244 77.5) (end 152.95 77.5) (width 0.2) (layer "F.Cu") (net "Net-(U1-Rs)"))
 (segment (start 154.1 111.209744) (end 154.415256 111.525) (width 0.2) (layer "F.Cu") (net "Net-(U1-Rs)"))
 (segment (start 152.95 77.5) (end 151.95 78.5) (width 0.2) (layer "F.Cu") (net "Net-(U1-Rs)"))
 (segment (start 154.415256 111.525) (end 155.384744 111.525) (width 0.2) (layer "F.Cu") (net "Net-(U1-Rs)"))
 (segment (start 161.3 105.609744) (end 161.3 101.811768) (width 0.2) (layer "F.Cu") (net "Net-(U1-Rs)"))
 (segment (start 155.384744 111.525) (end 161.3 105.609744) (width 0.2) (layer "F.Cu") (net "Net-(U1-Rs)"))
 (segment (start 154.1 109.790256) (end 154.1 111.209744) (width 0.2) (layer "F.Cu") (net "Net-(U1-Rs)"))
 (segment (start 136.925 97.595) (end 141.904744 97.595) (width 0.2) (layer "F.Cu") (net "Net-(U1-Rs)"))
 (segment (start 154.5875 77.815256) (end 154.272244 77.5) (width 0.2) (layer "F.Cu") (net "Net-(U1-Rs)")))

